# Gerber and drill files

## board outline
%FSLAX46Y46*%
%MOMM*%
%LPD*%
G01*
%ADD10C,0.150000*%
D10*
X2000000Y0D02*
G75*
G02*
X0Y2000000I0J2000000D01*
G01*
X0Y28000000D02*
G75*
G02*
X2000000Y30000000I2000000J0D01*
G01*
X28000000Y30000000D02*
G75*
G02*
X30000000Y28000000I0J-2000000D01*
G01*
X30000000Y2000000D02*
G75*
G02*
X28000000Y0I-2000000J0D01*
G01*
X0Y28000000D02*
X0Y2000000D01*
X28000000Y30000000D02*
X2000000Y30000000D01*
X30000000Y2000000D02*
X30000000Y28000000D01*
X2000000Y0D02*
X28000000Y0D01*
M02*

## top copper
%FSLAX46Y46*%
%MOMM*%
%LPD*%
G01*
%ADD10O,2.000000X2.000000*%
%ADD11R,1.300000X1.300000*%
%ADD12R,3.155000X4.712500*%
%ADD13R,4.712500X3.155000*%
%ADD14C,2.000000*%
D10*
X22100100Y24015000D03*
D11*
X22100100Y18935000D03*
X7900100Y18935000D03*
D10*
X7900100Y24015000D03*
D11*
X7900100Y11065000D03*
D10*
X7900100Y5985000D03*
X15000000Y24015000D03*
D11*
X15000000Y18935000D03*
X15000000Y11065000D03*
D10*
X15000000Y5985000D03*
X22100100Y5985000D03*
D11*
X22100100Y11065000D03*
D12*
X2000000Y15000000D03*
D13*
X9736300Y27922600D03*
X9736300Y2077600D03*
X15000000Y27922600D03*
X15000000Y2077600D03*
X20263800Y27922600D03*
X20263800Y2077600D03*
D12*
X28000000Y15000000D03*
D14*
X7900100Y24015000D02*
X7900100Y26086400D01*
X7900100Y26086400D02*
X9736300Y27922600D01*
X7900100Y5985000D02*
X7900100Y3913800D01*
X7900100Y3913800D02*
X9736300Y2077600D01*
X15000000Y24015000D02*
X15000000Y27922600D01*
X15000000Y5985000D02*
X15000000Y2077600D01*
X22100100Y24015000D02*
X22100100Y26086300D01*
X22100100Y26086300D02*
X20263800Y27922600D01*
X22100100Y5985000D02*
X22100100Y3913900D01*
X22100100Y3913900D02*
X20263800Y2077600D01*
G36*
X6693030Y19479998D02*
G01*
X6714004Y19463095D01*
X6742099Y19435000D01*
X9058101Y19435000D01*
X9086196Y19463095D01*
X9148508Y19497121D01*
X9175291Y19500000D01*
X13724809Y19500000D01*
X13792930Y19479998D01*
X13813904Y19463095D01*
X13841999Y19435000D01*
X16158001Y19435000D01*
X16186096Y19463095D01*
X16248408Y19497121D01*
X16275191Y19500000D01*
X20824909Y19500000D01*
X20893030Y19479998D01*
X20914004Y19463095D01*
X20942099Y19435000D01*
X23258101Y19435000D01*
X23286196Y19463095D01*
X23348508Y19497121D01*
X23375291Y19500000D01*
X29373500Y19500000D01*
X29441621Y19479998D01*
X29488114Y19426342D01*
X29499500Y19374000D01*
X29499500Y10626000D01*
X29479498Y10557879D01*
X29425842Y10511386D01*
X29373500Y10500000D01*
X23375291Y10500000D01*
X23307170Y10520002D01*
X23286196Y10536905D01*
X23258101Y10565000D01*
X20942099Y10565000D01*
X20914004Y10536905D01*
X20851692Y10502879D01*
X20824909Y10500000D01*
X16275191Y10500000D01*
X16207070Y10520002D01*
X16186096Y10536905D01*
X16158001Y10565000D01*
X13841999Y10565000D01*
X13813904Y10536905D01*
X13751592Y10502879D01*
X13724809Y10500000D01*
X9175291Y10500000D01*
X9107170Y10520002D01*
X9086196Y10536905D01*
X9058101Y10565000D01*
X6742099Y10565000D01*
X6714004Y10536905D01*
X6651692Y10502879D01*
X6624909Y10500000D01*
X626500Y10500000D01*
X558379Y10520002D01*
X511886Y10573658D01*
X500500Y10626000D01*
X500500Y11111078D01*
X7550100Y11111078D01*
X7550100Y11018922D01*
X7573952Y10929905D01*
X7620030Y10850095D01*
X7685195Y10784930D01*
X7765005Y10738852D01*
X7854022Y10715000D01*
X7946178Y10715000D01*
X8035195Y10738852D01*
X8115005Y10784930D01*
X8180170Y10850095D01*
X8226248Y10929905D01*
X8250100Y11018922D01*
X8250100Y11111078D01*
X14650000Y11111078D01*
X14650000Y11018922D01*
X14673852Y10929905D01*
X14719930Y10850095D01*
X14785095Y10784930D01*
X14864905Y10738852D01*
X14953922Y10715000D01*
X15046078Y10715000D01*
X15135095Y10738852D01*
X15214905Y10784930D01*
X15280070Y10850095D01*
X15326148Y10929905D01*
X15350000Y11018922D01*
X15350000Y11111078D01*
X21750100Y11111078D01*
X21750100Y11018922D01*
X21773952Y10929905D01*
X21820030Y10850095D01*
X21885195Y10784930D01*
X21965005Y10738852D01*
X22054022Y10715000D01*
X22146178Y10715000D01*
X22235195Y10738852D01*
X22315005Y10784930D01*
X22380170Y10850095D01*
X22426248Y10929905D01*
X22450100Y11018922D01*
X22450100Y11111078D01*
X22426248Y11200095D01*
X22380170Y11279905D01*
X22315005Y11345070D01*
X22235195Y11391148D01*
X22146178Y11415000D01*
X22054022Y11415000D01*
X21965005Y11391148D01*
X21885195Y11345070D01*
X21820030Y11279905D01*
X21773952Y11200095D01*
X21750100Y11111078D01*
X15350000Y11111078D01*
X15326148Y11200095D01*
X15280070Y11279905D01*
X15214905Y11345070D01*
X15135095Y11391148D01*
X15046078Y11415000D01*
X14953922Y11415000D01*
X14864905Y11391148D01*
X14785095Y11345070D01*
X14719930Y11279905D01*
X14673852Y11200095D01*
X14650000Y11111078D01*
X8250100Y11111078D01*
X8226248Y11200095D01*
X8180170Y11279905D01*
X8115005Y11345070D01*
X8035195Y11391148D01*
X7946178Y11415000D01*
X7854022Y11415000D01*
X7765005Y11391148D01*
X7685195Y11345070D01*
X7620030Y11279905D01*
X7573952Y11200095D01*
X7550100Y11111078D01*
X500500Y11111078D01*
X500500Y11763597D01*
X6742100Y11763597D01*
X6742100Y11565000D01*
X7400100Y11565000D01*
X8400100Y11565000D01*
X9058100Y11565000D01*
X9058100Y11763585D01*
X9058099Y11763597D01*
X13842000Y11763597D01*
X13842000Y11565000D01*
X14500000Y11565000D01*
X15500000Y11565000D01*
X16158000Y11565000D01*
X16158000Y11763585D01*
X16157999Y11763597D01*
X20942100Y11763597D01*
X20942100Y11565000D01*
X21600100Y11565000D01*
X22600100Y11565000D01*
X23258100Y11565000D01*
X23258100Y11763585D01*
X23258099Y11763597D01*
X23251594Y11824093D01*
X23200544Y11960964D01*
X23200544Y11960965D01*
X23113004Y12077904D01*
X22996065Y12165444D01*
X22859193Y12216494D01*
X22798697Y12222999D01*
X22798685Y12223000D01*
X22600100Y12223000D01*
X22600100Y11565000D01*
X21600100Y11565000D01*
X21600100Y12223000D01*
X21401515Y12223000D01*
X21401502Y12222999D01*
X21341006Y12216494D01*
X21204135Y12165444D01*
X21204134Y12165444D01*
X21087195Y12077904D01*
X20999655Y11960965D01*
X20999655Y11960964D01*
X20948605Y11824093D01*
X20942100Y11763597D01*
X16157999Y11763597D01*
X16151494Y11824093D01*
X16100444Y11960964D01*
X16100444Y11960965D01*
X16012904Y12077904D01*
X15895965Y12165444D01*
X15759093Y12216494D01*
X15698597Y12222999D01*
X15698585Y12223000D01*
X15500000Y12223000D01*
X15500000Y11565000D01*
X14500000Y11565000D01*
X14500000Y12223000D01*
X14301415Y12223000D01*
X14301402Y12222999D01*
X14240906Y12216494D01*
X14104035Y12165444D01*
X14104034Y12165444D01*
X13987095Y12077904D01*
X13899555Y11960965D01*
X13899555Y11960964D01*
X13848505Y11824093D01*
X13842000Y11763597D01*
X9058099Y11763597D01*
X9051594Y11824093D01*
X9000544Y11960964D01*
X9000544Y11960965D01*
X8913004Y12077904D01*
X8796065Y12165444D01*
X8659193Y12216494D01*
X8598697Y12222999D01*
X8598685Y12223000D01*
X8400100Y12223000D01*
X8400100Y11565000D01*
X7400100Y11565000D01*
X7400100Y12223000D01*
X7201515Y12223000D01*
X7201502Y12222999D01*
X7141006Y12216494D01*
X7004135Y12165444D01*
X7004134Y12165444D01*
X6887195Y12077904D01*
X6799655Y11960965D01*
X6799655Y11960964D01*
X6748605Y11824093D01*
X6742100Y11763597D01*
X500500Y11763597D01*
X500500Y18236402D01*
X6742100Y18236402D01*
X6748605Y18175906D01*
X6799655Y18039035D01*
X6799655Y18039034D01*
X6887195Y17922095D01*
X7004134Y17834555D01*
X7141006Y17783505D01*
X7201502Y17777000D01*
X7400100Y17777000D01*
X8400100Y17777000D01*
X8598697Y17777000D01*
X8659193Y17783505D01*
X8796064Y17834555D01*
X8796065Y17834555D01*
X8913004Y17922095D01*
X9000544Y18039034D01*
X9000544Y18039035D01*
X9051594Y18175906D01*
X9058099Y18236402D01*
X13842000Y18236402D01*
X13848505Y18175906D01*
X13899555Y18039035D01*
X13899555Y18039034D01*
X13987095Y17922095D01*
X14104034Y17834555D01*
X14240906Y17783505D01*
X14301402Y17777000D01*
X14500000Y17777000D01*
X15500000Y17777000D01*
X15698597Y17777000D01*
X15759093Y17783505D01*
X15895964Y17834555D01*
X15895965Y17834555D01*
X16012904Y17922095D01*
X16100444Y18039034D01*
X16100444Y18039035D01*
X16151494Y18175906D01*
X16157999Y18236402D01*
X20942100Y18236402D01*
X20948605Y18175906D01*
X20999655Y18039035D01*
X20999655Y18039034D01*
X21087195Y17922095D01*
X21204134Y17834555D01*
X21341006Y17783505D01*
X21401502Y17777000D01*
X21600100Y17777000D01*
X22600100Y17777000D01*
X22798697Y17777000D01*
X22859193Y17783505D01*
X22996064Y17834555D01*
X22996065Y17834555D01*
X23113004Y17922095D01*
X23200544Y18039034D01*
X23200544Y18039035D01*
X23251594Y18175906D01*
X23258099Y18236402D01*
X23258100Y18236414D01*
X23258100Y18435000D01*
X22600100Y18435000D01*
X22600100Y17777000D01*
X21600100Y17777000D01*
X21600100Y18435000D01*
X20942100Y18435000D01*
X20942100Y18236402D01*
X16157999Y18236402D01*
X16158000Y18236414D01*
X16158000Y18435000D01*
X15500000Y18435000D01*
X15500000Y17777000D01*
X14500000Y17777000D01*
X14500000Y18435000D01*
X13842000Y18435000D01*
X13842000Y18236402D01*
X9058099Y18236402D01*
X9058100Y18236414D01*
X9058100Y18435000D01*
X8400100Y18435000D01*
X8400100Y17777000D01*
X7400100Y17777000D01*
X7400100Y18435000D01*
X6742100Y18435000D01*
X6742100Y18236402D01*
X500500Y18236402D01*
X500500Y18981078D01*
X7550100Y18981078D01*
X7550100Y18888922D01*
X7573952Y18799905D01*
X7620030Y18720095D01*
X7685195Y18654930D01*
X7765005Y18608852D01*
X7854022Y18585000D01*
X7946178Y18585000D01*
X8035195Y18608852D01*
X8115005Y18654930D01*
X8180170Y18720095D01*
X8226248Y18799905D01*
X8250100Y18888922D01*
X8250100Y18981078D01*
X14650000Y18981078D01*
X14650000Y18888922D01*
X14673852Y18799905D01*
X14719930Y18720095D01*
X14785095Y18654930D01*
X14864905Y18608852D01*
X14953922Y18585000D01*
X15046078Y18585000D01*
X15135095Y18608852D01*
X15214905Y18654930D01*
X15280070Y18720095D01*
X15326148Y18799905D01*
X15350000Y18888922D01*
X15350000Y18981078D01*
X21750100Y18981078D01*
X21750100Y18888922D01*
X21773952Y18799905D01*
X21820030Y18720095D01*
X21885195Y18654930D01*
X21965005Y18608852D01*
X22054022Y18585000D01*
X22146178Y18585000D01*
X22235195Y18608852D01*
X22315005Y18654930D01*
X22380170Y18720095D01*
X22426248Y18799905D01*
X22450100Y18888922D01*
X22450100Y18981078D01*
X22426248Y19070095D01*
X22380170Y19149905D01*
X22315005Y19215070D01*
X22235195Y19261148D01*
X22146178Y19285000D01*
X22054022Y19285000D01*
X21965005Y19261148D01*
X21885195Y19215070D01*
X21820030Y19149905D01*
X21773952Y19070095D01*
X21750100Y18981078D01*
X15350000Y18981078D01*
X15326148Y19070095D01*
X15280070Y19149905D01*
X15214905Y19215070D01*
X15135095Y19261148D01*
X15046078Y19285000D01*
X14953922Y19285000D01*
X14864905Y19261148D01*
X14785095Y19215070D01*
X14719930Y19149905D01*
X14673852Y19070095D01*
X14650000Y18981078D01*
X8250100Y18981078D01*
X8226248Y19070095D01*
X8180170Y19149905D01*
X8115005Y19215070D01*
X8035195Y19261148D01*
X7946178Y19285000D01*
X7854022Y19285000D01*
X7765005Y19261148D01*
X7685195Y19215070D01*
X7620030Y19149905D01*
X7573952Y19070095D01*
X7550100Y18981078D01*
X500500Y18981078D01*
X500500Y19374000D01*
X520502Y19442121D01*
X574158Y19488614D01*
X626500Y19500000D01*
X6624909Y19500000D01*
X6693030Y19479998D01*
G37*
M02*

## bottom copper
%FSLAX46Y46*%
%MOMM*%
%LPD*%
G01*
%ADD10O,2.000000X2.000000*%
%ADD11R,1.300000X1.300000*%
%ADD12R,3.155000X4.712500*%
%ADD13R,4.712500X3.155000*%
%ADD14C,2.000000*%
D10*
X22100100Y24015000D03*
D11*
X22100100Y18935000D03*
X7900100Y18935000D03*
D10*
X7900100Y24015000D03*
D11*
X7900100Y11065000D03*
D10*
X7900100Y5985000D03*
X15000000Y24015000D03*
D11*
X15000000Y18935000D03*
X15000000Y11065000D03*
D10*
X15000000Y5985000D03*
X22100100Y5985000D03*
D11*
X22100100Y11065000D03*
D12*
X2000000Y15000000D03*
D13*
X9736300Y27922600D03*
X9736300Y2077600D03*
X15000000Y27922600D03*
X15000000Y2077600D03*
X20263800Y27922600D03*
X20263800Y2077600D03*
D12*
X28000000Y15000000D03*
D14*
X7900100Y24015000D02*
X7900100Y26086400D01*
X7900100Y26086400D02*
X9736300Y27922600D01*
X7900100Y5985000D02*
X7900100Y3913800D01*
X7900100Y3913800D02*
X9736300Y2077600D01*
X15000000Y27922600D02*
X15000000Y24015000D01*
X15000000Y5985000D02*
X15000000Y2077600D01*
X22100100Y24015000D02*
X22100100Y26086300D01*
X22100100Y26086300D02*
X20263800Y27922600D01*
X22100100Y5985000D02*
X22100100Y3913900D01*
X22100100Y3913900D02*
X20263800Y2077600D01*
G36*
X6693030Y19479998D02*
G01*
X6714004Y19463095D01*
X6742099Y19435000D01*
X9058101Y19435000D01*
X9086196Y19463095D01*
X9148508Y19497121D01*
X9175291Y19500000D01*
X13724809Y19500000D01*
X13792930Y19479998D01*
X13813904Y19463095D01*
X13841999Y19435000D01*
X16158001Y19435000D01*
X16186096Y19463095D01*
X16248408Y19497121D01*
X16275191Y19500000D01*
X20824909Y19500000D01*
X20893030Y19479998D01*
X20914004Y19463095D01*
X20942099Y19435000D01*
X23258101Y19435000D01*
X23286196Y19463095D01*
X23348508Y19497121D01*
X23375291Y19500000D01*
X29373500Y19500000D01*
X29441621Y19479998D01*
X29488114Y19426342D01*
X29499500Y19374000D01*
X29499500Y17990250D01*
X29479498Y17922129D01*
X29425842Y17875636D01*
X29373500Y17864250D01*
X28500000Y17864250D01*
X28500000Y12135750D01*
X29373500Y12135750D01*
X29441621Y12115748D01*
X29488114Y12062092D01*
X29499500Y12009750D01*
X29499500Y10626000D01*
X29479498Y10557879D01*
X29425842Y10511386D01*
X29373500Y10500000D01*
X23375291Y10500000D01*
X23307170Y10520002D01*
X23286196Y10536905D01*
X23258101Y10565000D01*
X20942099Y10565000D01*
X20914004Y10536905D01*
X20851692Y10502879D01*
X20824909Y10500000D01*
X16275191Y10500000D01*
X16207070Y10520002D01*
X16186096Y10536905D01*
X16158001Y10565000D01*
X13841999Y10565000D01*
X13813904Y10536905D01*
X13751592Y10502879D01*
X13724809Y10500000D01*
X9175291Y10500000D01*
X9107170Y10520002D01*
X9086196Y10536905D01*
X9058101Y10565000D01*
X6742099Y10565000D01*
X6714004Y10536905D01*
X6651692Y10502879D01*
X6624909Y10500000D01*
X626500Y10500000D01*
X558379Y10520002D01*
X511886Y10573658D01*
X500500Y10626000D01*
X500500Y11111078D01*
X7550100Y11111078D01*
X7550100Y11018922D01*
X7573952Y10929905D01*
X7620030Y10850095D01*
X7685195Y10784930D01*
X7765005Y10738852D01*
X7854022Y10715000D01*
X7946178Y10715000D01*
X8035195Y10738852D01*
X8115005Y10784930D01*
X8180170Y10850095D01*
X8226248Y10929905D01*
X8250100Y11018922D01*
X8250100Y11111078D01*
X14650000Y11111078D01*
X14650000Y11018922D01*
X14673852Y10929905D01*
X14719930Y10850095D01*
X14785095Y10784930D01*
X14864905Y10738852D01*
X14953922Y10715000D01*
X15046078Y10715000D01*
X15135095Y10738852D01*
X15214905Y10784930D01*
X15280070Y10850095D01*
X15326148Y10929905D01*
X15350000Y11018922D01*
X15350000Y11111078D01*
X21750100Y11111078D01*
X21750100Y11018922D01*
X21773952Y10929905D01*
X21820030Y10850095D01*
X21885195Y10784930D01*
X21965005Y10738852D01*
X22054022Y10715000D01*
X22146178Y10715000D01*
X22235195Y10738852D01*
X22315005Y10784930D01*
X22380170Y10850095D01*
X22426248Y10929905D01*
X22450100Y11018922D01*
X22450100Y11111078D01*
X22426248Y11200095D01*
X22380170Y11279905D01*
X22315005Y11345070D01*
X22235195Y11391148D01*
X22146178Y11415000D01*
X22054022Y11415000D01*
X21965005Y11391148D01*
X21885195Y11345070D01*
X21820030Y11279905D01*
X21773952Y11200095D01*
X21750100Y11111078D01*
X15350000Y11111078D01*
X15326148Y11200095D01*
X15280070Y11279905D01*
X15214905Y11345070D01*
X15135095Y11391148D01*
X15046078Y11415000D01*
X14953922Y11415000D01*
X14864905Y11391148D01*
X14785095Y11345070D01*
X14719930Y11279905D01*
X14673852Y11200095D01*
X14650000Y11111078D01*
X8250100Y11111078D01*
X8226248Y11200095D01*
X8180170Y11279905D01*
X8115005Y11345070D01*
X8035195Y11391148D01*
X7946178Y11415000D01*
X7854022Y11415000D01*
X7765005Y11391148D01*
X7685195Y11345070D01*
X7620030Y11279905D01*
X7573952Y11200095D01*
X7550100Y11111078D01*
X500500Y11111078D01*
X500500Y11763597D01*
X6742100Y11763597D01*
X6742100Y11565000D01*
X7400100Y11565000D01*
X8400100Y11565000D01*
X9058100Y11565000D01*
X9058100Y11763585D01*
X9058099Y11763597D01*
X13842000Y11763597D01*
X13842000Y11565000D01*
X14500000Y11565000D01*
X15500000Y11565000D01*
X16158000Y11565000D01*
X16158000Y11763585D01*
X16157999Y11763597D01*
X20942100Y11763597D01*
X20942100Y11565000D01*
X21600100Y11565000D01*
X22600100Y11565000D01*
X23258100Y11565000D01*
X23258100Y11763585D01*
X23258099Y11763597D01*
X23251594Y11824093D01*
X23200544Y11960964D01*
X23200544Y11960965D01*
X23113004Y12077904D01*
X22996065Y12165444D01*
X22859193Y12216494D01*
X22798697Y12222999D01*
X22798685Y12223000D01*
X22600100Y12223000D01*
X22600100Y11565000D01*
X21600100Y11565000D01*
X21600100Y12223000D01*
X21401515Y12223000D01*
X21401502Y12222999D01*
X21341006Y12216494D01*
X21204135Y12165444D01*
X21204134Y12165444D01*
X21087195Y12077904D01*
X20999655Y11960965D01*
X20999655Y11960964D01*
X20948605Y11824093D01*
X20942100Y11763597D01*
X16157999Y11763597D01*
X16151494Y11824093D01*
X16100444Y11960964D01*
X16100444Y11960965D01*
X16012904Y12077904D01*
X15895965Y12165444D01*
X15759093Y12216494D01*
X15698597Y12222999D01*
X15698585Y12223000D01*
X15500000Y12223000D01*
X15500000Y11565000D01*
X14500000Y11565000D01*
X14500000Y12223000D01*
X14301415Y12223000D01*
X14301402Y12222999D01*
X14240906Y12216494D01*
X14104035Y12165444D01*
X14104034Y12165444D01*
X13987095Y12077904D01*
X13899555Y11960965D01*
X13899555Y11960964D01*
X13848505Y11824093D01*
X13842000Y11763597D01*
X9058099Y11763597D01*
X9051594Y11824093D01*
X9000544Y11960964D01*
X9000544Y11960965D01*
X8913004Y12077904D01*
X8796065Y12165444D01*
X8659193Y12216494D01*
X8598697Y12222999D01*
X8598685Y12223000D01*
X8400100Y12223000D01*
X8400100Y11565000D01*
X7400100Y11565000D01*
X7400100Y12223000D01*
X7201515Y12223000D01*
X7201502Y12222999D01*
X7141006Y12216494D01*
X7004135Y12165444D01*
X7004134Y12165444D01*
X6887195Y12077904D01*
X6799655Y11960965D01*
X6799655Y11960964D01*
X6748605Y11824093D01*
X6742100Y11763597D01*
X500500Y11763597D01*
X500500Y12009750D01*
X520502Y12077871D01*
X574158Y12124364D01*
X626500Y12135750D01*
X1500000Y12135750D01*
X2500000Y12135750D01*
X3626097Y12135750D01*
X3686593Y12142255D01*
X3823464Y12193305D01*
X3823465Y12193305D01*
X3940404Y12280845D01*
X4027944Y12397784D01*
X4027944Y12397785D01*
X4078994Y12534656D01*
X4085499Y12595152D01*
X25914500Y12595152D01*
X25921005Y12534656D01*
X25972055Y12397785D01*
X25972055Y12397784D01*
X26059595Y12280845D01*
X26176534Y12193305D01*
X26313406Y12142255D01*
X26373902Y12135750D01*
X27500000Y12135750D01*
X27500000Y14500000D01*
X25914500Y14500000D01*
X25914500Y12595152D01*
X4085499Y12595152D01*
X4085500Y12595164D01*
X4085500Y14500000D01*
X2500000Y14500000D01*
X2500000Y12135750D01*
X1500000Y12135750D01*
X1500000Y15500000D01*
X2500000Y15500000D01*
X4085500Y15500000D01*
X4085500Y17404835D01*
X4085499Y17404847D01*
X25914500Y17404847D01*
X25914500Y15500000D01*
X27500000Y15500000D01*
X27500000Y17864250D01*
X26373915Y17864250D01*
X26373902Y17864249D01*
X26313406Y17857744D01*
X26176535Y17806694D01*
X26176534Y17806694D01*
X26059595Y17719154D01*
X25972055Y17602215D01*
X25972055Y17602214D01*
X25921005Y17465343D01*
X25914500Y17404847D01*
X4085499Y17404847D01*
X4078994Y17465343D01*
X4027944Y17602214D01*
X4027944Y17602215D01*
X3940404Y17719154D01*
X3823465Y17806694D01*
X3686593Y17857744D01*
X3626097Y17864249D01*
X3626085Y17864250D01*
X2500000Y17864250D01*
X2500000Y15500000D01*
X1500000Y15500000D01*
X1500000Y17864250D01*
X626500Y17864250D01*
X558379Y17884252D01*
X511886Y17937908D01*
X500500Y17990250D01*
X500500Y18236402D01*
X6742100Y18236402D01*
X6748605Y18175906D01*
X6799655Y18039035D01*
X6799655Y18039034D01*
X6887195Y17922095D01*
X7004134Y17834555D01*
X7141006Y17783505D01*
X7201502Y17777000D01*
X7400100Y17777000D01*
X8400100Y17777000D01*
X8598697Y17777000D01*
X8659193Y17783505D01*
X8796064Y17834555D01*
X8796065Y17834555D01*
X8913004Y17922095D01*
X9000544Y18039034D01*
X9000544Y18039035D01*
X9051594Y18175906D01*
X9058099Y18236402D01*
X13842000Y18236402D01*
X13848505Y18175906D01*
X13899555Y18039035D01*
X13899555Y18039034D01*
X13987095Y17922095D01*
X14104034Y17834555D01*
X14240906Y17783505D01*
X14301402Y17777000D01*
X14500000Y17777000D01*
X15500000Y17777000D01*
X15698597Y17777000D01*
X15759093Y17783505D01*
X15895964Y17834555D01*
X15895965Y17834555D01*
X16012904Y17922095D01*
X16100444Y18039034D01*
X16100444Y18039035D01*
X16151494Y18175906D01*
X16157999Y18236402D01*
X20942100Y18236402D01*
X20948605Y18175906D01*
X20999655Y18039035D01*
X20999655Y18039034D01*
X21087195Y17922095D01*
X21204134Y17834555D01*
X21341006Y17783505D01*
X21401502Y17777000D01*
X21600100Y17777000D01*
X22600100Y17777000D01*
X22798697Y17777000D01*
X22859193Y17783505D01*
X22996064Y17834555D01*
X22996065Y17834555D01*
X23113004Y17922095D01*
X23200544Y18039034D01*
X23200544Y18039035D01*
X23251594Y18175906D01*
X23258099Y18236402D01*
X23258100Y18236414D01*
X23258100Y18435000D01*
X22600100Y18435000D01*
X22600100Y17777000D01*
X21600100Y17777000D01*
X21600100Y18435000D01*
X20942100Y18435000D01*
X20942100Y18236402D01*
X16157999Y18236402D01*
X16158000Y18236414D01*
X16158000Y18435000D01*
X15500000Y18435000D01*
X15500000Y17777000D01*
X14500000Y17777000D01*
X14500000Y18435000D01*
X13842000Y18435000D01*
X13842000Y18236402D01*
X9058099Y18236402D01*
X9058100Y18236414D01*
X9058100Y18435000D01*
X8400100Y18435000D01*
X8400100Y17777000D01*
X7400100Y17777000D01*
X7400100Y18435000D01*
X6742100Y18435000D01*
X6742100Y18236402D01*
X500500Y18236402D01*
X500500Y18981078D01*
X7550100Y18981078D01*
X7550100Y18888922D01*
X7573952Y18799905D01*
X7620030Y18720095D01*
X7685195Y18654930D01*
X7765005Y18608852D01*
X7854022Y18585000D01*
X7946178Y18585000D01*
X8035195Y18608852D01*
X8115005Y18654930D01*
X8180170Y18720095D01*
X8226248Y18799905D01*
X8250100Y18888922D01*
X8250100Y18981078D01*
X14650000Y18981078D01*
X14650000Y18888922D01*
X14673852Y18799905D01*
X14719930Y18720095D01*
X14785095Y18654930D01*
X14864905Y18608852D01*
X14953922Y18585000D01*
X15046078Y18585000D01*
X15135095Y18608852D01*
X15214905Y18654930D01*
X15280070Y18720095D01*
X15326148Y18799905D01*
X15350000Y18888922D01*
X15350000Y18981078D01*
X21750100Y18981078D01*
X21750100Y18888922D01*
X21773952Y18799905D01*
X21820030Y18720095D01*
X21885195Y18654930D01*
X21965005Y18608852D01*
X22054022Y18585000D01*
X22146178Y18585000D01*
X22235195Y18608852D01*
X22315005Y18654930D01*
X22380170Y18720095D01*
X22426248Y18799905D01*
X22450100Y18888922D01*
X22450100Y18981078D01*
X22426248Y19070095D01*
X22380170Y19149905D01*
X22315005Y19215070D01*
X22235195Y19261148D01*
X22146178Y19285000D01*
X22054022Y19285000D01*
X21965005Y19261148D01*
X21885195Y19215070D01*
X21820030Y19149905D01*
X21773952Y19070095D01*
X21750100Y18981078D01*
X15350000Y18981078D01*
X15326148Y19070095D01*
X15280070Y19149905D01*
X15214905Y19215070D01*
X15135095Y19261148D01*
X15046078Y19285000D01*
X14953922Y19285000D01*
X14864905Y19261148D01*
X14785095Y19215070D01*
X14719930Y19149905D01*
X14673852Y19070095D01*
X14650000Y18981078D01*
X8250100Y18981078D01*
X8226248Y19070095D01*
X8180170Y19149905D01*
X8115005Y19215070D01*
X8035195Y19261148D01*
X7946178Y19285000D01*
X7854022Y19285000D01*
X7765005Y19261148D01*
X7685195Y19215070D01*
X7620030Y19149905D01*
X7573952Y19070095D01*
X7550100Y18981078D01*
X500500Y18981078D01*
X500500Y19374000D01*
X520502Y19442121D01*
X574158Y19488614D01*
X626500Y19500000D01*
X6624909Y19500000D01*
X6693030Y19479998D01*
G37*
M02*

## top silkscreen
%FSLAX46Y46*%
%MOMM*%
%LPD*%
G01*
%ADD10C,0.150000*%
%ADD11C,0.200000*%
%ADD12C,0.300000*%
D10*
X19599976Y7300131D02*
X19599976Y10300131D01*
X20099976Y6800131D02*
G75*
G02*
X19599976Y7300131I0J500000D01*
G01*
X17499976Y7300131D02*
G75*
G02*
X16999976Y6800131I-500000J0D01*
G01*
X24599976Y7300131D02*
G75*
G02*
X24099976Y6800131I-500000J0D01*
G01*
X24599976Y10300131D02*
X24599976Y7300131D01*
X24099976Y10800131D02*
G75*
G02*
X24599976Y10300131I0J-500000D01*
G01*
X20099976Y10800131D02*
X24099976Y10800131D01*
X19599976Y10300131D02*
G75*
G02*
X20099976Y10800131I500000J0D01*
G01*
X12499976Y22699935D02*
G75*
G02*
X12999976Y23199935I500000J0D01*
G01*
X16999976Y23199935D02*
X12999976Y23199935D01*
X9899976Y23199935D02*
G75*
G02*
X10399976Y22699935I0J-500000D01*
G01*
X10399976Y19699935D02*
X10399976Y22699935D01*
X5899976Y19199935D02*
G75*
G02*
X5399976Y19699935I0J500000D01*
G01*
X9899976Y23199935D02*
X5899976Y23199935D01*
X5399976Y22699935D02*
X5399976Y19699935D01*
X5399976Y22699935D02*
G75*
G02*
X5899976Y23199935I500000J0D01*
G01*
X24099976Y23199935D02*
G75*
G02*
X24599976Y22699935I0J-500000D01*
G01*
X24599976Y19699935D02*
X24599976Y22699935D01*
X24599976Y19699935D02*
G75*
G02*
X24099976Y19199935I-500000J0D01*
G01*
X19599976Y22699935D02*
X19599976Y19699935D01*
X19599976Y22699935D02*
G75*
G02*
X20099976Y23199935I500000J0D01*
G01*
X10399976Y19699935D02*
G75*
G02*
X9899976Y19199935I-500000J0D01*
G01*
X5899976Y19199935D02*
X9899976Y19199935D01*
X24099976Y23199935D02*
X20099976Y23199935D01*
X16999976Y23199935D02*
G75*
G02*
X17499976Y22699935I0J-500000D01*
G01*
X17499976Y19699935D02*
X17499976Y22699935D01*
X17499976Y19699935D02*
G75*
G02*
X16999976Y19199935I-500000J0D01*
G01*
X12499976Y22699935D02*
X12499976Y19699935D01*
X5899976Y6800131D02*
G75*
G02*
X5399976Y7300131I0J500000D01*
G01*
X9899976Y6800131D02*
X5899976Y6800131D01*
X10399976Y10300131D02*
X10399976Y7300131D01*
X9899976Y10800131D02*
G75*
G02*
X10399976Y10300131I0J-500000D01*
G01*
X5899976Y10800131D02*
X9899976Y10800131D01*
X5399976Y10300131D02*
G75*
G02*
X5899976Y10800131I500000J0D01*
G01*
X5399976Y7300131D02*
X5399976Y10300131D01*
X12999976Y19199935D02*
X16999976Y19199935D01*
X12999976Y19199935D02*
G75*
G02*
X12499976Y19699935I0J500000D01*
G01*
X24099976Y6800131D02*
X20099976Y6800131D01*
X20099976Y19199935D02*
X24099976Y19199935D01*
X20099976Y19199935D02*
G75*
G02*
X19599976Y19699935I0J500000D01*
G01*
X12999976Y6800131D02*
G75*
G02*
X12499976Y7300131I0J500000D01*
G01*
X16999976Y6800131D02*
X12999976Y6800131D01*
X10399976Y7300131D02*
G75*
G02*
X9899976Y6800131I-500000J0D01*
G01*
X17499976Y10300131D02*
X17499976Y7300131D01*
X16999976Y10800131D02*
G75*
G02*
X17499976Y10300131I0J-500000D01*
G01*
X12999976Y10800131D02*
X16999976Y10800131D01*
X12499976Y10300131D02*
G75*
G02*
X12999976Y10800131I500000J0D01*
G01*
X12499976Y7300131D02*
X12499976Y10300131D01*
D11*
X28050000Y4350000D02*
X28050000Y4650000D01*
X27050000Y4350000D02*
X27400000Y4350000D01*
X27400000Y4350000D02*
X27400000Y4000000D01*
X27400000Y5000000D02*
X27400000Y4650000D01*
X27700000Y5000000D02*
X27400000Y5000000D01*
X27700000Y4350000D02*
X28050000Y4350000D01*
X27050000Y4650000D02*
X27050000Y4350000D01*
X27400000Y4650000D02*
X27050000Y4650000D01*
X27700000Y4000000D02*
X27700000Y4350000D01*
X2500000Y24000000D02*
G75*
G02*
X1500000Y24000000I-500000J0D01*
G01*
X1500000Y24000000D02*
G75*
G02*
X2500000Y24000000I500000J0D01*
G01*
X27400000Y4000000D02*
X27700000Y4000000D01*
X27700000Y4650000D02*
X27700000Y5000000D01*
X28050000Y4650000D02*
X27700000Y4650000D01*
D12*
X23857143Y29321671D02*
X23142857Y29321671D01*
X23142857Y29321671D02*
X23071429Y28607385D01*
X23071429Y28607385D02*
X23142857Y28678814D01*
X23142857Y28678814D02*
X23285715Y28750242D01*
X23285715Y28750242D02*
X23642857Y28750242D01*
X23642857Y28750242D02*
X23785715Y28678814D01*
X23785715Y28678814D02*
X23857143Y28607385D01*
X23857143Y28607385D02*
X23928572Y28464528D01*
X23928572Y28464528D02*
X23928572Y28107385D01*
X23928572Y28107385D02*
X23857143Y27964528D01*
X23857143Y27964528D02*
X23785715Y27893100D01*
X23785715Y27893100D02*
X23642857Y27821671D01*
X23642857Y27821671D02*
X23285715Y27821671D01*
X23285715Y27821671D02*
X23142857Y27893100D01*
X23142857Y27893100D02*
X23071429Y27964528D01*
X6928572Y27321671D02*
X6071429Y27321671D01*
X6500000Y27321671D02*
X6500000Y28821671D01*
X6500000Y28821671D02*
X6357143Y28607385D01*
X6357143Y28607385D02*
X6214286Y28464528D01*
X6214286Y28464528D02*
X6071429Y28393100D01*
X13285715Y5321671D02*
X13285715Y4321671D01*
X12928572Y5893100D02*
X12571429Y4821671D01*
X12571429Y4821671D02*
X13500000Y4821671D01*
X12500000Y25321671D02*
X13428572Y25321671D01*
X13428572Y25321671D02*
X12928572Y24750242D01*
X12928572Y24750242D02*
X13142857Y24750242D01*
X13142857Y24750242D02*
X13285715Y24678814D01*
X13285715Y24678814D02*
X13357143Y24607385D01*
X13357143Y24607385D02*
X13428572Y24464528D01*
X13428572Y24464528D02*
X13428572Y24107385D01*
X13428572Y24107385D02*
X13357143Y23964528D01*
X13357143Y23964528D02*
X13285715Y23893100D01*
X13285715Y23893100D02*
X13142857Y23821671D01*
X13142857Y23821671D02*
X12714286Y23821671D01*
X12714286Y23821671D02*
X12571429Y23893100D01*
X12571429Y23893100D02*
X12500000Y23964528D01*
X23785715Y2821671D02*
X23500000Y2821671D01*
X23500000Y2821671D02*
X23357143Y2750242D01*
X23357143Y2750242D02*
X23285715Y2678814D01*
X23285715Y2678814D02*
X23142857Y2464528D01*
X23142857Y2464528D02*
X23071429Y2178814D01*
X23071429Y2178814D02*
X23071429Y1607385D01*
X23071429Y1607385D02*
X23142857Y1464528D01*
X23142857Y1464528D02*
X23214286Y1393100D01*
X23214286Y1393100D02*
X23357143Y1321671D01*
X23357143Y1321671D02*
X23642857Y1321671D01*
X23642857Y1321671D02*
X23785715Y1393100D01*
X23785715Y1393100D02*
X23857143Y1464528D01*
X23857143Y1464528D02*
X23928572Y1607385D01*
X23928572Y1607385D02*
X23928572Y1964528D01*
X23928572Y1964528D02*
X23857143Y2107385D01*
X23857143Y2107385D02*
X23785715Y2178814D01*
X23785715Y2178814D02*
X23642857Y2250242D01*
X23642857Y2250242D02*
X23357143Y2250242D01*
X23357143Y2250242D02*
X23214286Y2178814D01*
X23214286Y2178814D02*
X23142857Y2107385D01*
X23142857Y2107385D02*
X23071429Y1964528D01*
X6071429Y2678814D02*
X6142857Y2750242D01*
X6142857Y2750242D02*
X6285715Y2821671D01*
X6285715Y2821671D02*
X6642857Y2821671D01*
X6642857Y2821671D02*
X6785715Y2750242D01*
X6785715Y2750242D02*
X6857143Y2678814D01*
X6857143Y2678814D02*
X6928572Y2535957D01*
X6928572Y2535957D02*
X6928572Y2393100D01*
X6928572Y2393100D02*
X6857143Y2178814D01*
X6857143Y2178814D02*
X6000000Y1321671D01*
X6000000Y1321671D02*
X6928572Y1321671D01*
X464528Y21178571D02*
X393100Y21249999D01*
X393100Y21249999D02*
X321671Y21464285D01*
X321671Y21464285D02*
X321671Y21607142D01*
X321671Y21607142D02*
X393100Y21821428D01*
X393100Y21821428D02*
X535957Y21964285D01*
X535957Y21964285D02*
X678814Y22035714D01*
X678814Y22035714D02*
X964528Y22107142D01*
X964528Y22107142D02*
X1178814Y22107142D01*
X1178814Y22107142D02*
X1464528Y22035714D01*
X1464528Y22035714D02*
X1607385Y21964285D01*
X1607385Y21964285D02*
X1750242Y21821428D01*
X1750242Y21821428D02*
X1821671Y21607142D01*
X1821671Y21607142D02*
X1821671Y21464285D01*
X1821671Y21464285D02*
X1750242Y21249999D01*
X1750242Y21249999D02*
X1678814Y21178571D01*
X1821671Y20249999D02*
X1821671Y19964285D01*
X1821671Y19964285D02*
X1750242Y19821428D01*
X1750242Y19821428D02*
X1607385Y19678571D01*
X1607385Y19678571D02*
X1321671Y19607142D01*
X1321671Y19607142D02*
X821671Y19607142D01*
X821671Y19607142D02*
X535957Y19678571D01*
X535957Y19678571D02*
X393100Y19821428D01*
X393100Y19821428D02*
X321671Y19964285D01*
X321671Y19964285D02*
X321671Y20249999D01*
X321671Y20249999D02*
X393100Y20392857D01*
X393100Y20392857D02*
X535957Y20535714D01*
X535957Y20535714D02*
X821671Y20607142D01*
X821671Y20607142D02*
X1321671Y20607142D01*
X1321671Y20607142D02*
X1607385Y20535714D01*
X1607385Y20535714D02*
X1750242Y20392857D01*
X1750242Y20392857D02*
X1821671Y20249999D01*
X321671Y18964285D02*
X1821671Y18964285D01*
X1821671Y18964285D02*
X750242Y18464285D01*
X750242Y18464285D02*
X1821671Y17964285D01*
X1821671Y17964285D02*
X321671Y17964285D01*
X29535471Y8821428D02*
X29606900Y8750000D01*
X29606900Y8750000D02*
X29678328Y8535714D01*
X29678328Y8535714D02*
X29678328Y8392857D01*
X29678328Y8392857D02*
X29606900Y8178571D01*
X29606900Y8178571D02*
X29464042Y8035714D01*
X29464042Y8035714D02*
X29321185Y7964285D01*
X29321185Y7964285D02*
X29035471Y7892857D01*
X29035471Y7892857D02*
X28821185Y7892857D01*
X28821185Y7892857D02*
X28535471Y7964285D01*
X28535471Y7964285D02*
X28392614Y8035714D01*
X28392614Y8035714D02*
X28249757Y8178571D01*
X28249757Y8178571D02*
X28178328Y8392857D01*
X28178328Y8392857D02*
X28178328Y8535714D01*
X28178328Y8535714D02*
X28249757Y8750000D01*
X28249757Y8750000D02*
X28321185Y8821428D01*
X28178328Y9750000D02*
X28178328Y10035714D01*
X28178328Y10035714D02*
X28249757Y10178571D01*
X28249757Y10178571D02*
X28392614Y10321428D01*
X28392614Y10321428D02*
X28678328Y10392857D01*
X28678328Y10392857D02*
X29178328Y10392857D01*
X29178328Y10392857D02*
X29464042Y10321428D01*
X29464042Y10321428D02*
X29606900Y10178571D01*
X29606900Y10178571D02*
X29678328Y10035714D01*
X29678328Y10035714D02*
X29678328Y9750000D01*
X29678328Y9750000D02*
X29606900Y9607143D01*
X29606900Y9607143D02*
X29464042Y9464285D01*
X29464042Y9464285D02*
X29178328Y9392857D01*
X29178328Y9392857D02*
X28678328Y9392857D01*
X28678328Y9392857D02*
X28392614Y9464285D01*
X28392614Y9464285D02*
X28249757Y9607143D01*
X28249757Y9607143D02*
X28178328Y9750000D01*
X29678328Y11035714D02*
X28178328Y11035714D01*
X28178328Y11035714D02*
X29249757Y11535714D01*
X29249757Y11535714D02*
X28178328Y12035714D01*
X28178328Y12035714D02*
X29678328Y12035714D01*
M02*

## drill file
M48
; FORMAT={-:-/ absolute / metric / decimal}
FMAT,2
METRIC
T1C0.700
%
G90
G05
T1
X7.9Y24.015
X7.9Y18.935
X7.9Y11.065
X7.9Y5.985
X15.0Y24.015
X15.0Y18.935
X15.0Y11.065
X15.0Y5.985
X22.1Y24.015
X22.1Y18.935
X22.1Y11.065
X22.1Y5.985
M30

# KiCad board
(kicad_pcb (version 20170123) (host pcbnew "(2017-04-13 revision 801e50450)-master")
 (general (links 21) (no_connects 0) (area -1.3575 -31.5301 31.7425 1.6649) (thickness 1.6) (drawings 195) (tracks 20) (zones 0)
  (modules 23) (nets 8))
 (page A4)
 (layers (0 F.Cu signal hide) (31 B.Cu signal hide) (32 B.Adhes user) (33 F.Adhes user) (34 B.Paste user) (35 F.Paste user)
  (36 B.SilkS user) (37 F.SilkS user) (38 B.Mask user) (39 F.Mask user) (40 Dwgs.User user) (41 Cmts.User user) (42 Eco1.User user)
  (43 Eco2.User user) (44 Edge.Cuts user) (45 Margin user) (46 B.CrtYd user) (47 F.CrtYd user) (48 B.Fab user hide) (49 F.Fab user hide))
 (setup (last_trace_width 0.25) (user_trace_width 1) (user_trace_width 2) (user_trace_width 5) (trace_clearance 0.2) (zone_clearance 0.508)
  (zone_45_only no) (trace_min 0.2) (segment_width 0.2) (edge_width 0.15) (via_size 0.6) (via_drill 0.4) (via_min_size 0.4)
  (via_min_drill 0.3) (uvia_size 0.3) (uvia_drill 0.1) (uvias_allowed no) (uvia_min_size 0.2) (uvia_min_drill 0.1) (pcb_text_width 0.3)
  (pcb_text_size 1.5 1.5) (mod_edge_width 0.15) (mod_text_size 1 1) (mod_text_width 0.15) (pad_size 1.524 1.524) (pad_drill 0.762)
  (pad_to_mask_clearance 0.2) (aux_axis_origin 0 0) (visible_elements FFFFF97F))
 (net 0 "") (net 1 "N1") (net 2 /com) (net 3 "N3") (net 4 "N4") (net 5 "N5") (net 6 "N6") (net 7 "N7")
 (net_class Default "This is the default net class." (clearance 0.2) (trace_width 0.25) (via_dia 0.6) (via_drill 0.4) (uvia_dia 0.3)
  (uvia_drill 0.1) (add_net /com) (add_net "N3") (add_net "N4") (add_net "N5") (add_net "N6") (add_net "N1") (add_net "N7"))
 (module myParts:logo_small (layer B.Cu) (at 15 -15)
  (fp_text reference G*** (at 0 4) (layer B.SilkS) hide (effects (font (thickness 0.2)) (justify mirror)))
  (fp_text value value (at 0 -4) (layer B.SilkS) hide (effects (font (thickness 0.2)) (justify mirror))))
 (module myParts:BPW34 (layer B.Cu) (at 22.1001 -18.935 90)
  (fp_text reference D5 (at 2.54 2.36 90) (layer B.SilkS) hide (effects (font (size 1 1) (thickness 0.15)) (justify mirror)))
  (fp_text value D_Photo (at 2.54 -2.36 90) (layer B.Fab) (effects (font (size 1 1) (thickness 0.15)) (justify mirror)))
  (pad 2 thru_hole oval (at 5.08 0 90) (size 2 2) (drill 0.7) (layers *.Cu *.Mask) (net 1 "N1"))
  (pad 1 thru_hole rect (at 0 0 90) (size 1.3 1.3) (drill 0.7) (layers *.Cu *.Mask) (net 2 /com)))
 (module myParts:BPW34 (layer B.Cu) (at 7.9001 -18.935 90)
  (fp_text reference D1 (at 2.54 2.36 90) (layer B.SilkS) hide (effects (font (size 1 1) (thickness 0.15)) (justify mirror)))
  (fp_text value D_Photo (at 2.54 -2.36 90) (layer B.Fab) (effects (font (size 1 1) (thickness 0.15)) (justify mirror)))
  (pad 1 thru_hole rect (at 0 0 90) (size 1.3 1.3) (drill 0.7) (layers *.Cu *.Mask) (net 2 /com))
  (pad 2 thru_hole oval (at 5.08 0 90) (size 2 2) (drill 0.7) (layers *.Cu *.Mask) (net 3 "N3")))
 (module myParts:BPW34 (layer B.Cu) (at 7.9001 -11.065 270)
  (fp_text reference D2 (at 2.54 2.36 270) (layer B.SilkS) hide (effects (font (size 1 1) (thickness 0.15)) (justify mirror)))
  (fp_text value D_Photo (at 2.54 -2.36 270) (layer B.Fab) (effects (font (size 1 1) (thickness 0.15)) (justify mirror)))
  (pad 1 thru_hole rect (at 0 0 270) (size 1.3 1.3) (drill 0.7) (layers *.Cu *.Mask) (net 2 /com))
  (pad 2 thru_hole oval (at 5.08 0 270) (size 2 2) (drill 0.7) (layers *.Cu *.Mask) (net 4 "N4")))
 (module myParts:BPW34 (layer B.Cu) (at 15 -18.935 90)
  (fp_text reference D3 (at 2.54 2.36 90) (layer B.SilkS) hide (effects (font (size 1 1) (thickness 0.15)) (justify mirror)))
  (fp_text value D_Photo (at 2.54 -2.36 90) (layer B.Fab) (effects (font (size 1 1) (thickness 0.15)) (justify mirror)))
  (pad 2 thru_hole oval (at 5.08 0 90) (size 2 2) (drill 0.7) (layers *.Cu *.Mask) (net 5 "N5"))
  (pad 1 thru_hole rect (at 0 0 90) (size 1.3 1.3) (drill 0.7) (layers *.Cu *.Mask) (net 2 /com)))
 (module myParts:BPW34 (layer B.Cu) (at 15 -11.065 270)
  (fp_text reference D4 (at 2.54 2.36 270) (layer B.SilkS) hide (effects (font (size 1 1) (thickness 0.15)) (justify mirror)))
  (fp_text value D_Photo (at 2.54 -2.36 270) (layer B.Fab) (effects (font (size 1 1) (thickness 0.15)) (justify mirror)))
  (pad 1 thru_hole rect (at 0 0 270) (size 1.3 1.3) (drill 0.7) (layers *.Cu *.Mask) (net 2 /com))
  (pad 2 thru_hole oval (at 5.08 0 270) (size 2 2) (drill 0.7) (layers *.Cu *.Mask) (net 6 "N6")))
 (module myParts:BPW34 (layer B.Cu) (at 22.1001 -11.065 270)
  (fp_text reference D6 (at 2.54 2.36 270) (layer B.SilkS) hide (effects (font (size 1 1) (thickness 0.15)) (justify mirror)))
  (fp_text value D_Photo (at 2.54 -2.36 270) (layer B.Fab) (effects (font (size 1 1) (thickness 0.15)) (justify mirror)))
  (pad 2 thru_hole oval (at 5.08 0 270) (size 2 2) (drill 0.7) (layers *.Cu *.Mask) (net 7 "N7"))
  (pad 1 thru_hole rect (at 0 0 270) (size 1.3 1.3) (drill 0.7) (layers *.Cu *.Mask) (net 2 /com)))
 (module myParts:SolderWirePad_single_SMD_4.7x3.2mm (layer F.Cu) (at 2 -15 90)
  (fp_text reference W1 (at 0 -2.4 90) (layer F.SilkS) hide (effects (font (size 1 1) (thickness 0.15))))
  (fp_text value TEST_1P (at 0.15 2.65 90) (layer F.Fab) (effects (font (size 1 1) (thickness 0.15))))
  (pad 1 smd rect (at 0 0 90) (size 4.7125 3.155) (layers F.Cu F.Paste F.Mask) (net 2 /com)))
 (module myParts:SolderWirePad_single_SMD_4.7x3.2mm (layer F.Cu) (at 9.7363 -27.9226)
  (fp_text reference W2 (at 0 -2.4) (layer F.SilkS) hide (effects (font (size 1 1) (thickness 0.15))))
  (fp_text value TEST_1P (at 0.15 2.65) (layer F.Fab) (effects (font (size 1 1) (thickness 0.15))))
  (pad 1 smd rect (at 0 0) (size 4.7125 3.155) (layers F.Cu F.Paste F.Mask) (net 3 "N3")))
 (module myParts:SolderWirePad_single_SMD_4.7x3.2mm (layer F.Cu) (at 9.7363 -2.0776)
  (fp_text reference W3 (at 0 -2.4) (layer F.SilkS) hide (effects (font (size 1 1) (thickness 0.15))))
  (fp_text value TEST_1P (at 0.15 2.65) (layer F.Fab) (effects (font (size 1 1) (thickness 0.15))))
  (pad 1 smd rect (at 0 0) (size 4.7125 3.155) (layers F.Cu F.Paste F.Mask) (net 4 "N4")))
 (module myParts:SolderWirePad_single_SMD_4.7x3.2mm (layer F.Cu) (at 15 -27.9226)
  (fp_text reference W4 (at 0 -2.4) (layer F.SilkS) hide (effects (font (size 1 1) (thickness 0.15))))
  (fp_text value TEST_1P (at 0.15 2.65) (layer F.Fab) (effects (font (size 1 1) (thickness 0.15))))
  (pad 1 smd rect (at 0 0) (size 4.7125 3.155) (layers F.Cu F.Paste F.Mask) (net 5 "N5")))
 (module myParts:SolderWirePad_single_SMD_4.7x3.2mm (layer F.Cu) (at 15 -2.0776)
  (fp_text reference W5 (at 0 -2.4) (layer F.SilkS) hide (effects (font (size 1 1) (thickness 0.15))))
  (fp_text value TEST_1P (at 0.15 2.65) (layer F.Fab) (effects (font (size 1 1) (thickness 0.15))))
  (pad 1 smd rect (at 0 0) (size 4.7125 3.155) (layers F.Cu F.Paste F.Mask) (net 6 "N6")))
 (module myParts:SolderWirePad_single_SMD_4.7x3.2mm (layer F.Cu) (at 20.2638 -27.9226)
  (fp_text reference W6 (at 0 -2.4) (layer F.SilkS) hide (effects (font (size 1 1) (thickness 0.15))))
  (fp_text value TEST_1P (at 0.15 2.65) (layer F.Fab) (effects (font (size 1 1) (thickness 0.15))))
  (pad 1 smd rect (at 0 0) (size 4.7125 3.155) (layers F.Cu F.Paste F.Mask) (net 1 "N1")))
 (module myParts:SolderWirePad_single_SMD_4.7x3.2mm (layer F.Cu) (at 20.2638 -2.0776)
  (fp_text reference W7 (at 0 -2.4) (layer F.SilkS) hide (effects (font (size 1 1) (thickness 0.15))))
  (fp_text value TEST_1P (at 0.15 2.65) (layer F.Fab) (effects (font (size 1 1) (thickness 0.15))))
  (pad 1 smd rect (at 0 0) (size 4.7125 3.155) (layers F.Cu F.Paste F.Mask) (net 7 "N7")))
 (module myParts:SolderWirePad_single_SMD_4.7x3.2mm (layer F.Cu) (at 28 -15 90)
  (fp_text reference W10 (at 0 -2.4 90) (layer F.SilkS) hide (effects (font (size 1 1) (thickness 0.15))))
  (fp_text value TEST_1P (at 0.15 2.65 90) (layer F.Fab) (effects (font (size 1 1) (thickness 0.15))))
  (pad 1 smd rect (at 0 0 90) (size 4.7125 3.155) (layers F.Cu F.Paste F.Mask) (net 2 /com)))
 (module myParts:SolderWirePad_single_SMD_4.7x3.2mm (layer B.Cu) (at 2 -15 270)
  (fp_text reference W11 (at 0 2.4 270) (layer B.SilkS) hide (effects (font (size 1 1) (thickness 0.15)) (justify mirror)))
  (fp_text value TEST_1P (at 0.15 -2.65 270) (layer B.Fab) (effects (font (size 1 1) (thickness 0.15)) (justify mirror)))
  (pad 1 smd rect (at 0 0 270) (size 4.7125 3.155) (layers B.Cu B.Paste B.Mask) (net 2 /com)))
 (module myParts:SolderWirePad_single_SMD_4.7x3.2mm (layer B.Cu) (at 9.7363 -27.9226)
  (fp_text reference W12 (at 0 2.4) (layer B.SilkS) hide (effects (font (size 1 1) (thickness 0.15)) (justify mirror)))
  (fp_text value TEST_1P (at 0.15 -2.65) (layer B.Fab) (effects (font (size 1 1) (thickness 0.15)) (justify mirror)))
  (pad 1 smd rect (at 0 0) (size 4.7125 3.155) (layers B.Cu B.Paste B.Mask) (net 3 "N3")))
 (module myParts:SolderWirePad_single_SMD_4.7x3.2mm (layer B.Cu) (at 9.7363 -2.0776)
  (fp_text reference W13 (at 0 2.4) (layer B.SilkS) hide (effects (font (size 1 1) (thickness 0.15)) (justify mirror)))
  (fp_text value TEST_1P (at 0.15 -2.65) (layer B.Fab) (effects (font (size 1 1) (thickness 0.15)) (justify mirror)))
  (pad 1 smd rect (at 0 0) (size 4.7125 3.155) (layers B.Cu B.Paste B.Mask) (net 4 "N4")))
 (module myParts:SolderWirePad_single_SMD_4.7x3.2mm (layer B.Cu) (at 15 -27.9226)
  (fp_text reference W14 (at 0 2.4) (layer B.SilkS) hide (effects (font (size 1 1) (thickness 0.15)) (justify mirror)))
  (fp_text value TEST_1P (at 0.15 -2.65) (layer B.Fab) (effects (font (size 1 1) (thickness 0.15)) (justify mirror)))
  (pad 1 smd rect (at 0 0) (size 4.7125 3.155) (layers B.Cu B.Paste B.Mask) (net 5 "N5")))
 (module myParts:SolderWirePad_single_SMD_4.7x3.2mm (layer B.Cu) (at 15 -2.0776)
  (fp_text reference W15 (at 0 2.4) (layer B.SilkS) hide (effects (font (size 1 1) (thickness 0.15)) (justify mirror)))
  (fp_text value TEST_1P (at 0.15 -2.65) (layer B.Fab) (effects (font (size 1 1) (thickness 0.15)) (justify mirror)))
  (pad 1 smd rect (at 0 0) (size 4.7125 3.155) (layers B.Cu B.Paste B.Mask) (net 6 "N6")))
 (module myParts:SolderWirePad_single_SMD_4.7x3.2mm (layer B.Cu) (at 20.2638 -27.9226)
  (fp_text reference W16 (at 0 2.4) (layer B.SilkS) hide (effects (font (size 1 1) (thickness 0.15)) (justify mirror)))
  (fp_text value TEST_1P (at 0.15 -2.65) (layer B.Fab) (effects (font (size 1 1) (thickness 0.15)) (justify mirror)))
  (pad 1 smd rect (at 0 0) (size 4.7125 3.155) (layers B.Cu B.Paste B.Mask) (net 1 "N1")))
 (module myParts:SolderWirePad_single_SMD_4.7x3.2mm (layer B.Cu) (at 20.2638 -2.0776)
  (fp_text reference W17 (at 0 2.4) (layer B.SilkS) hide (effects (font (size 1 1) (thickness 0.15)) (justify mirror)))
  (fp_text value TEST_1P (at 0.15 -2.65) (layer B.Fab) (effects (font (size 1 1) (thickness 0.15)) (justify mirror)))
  (pad 1 smd rect (at 0 0) (size 4.7125 3.155) (layers B.Cu B.Paste B.Mask) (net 7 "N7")))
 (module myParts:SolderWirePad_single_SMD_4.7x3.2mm (layer B.Cu) (at 28 -15 270)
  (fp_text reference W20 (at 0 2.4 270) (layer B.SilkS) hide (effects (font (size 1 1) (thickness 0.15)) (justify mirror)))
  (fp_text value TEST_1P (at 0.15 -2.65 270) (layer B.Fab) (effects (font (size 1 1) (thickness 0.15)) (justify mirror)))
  (pad 1 smd rect (at 0 0 270) (size 4.7125 3.155) (layers B.Cu B.Paste B.Mask) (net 2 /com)))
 (gr_line (start 19.599976 -7.300131) (end 19.599976 -10.300131) (layer F.SilkS) (width 0.15))
 (gr_arc (start 20.099976 -7.300131) (end 19.599976 -7.300131) (angle -90) (layer F.SilkS) (width 0.15))
 (gr_arc (start 16.999976 -7.300131) (end 16.999976 -6.800131) (angle -90) (layer F.SilkS) (width 0.15))
 (gr_arc (start 24.099976 -7.300131) (end 24.099976 -6.800131) (angle -90) (layer F.SilkS) (width 0.15))
 (gr_line (start 24.599976 -10.300131) (end 24.599976 -7.300131) (layer F.SilkS) (width 0.15))
 (gr_arc (start 24.099976 -10.300131) (end 24.599976 -10.300131) (angle -90) (layer F.SilkS) (width 0.15))
 (gr_line (start 20.099976 -10.800131) (end 24.099976 -10.800131) (layer F.SilkS) (width 0.15))
 (gr_arc (start 20.099976 -10.300131) (end 20.099976 -10.800131) (angle -90) (layer F.SilkS) (width 0.15))
 (gr_arc (start 12.999976 -22.699935) (end 12.999976 -23.199935) (angle -90) (layer F.SilkS) (width 0.15))
 (gr_line (start 16.999976 -23.199935) (end 12.999976 -23.199935) (layer F.SilkS) (width 0.15))
 (gr_arc (start 9.899976 -22.699935) (end 10.399976 -22.699935) (angle -90) (layer F.SilkS) (width 0.15))
 (gr_line (start 10.399976 -19.699935) (end 10.399976 -22.699935) (layer F.SilkS) (width 0.15))
 (gr_arc (start 5.899976 -19.699935) (end 5.399976 -19.699935) (angle -90) (layer F.SilkS) (width 0.15))
 (gr_line (start 9.899976 -23.199935) (end 5.899976 -23.199935) (layer F.SilkS) (width 0.15))
 (gr_line (start 5.399976 -22.699935) (end 5.399976 -19.699935) (layer F.SilkS) (width 0.15))
 (gr_arc (start 5.899976 -22.699935) (end 5.899976 -23.199935) (angle -90) (layer F.SilkS) (width 0.15))
 (gr_arc (start 24.099976 -22.699935) (end 24.599976 -22.699935) (angle -90) (layer F.SilkS) (width 0.15))
 (gr_line (start 24.599976 -19.699935) (end 24.599976 -22.699935) (layer F.SilkS) (width 0.15))
 (gr_arc (start 24.099976 -19.699935) (end 24.099976 -19.199935) (angle -90) (layer F.SilkS) (width 0.15))
 (gr_line (start 19.599976 -22.699935) (end 19.599976 -19.699935) (layer F.SilkS) (width 0.15))
 (gr_arc (start 20.099976 -22.699935) (end 20.099976 -23.199935) (angle -90) (layer F.SilkS) (width 0.15))
 (gr_arc (start 9.899976 -19.699935) (end 9.899976 -19.199935) (angle -90) (layer F.SilkS) (width 0.15))
 (gr_line (start 5.899976 -19.199935) (end 9.899976 -19.199935) (layer F.SilkS) (width 0.15))
 (gr_line (start 24.099976 -23.199935) (end 20.099976 -23.199935) (layer F.SilkS) (width 0.15))
 (gr_arc (start 16.999976 -22.699935) (end 17.499976 -22.699935) (angle -90) (layer F.SilkS) (width 0.15))
 (gr_line (start 17.499976 -19.699935) (end 17.499976 -22.699935) (layer F.SilkS) (width 0.15))
 (gr_arc (start 16.999976 -19.699935) (end 16.999976 -19.199935) (angle -90) (layer F.SilkS) (width 0.15))
 (gr_line (start 12.499976 -22.699935) (end 12.499976 -19.699935) (layer F.SilkS) (width 0.15))
 (gr_arc (start 5.899976 -7.300131) (end 5.399976 -7.300131) (angle -90) (layer F.SilkS) (width 0.15))
 (gr_line (start 9.899976 -6.800131) (end 5.899976 -6.800131) (layer F.SilkS) (width 0.15))
 (gr_line (start 10.399976 -10.300131) (end 10.399976 -7.300131) (layer F.SilkS) (width 0.15))
 (gr_arc (start 9.899976 -10.300131) (end 10.399976 -10.300131) (angle -90) (layer F.SilkS) (width 0.15))
 (gr_line (start 5.899976 -10.800131) (end 9.899976 -10.800131) (layer F.SilkS) (width 0.15))
 (gr_arc (start 5.899976 -10.300131) (end 5.899976 -10.800131) (angle -90) (layer F.SilkS) (width 0.15))
 (gr_line (start 5.399976 -7.300131) (end 5.399976 -10.300131) (layer F.SilkS) (width 0.15))
 (gr_line (start 12.999976 -19.199935) (end 16.999976 -19.199935) (layer F.SilkS) (width 0.15))
 (gr_arc (start 12.999976 -19.699935) (end 12.499976 -19.699935) (angle -90) (layer F.SilkS) (width 0.15))
 (gr_line (start 24.099976 -6.800131) (end 20.099976 -6.800131) (layer F.SilkS) (width 0.15))
 (gr_line (start 20.099976 -19.199935) (end 24.099976 -19.199935) (layer F.SilkS) (width 0.15))
 (gr_arc (start 20.099976 -19.699935) (end 19.599976 -19.699935) (angle -90) (layer F.SilkS) (width 0.15))
 (gr_arc (start 12.999976 -7.300131) (end 12.499976 -7.300131) (angle -90) (layer F.SilkS) (width 0.15))
 (gr_line (start 16.999976 -6.800131) (end 12.999976 -6.800131) (layer F.SilkS) (width 0.15))
 (gr_arc (start 9.899976 -7.300131) (end 9.899976 -6.800131) (angle -90) (layer F.SilkS) (width 0.15))
 (gr_line (start 17.499976 -10.300131) (end 17.499976 -7.300131) (layer F.SilkS) (width 0.15))
 (gr_arc (start 16.999976 -10.300131) (end 17.499976 -10.300131) (angle -90) (layer F.SilkS) (width 0.15))
 (gr_line (start 12.999976 -10.800131) (end 16.999976 -10.800131) (layer F.SilkS) (width 0.15))
 (gr_arc (start 12.999976 -10.300131) (end 12.999976 -10.800131) (angle -90) (layer F.SilkS) (width 0.15))
 (gr_line (start 12.499976 -7.300131) (end 12.499976 -10.300131) (layer F.SilkS) (width 0.15))
 (gr_line (start 28.05 -4.35) (end 28.05 -4.65) (layer F.SilkS) (width 0.2))
 (gr_line (start 27.05 -4.35) (end 27.4 -4.35) (layer F.SilkS) (width 0.2))
 (gr_line (start 27.4 -4.35) (end 27.4 -4) (layer F.SilkS) (width 0.2))
 (gr_line (start 27.4 -5) (end 27.4 -4.65) (layer F.SilkS) (width 0.2))
 (gr_line (start 27.7 -5) (end 27.4 -5) (layer F.SilkS) (width 0.2))
 (gr_line (start 27.7 -4.35) (end 28.05 -4.35) (layer F.SilkS) (width 0.2))
 (gr_line (start 27.05 -4.65) (end 27.05 -4.35) (layer F.SilkS) (width 0.2))
 (gr_line (start 27.4 -4.65) (end 27.05 -4.65) (layer F.SilkS) (width 0.2))
 (gr_line (start 27.7 -4) (end 27.7 -4.35) (layer F.SilkS) (width 0.2))
 (gr_circle (center 2 -24) (end 2.5 -24) (layer F.SilkS) (width 0.2))
 (gr_line (start 27.4 -4) (end 27.7 -4) (layer F.SilkS) (width 0.2))
 (gr_line (start 27.7 -4.65) (end 27.7 -5) (layer F.SilkS) (width 0.2))
 (gr_line (start 28.05 -4.65) (end 27.7 -4.65) (layer F.SilkS) (width 0.2))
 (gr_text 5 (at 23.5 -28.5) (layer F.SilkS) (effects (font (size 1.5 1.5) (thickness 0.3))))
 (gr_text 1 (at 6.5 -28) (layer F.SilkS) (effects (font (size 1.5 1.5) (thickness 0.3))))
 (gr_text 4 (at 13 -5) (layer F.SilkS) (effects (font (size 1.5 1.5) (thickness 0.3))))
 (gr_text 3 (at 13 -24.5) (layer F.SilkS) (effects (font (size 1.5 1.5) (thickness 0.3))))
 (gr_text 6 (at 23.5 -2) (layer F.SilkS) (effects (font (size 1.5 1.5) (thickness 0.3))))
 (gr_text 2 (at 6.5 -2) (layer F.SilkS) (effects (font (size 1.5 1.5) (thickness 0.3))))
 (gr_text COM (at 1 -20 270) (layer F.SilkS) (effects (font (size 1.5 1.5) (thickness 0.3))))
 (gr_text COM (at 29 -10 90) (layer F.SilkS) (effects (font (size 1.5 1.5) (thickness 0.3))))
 (gr_arc (start 2 -2) (end 2 0) (angle 90) (layer Edge.Cuts) (width 0.15))
 (gr_arc (start 2 -28) (end 0 -28) (angle 90) (layer Edge.Cuts) (width 0.15))
 (gr_arc (start 28 -28) (end 28 -30) (angle 90) (layer Edge.Cuts) (width 0.15))
 (gr_arc (start 28 -2) (end 30 -2) (angle 90) (layer Edge.Cuts) (width 0.15))
 (gr_line (start 0 -28) (end 0 -2) (layer Edge.Cuts) (width 0.15))
 (gr_line (start 28 -30) (end 2 -30) (layer Edge.Cuts) (width 0.15))
 (gr_line (start 30 -2) (end 30 -28) (layer Edge.Cuts) (width 0.15))
 (gr_line (start 2 0) (end 28 0) (layer Edge.Cuts) (width 0.15))
 (segment (start 7.9001 -24.015) (end 7.9001 -26.0864) (width 2) (layer F.Cu) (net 3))
 (segment (start 7.9001 -26.0864) (end 9.7363 -27.9226) (width 2) (layer F.Cu) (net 3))
 (segment (start 7.9001 -24.015) (end 7.9001 -26.0864) (width 2) (layer B.Cu) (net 3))
 (segment (start 7.9001 -26.0864) (end 9.7363 -27.9226) (width 2) (layer B.Cu) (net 3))
 (segment (start 7.9001 -5.985) (end 7.9001 -3.9138) (width 2) (layer B.Cu) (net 4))
 (segment (start 7.9001 -3.9138) (end 9.7363 -2.0776) (width 2) (layer B.Cu) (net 4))
 (segment (start 7.9001 -5.985) (end 7.9001 -3.9138) (width 2) (layer F.Cu) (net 4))
 (segment (start 7.9001 -3.9138) (end 9.7363 -2.0776) (width 2) (layer F.Cu) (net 4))
 (segment (start 15 -24.015) (end 15 -27.9226) (width 2) (layer F.Cu) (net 5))
 (segment (start 15 -27.9226) (end 15 -24.015) (width 2) (layer B.Cu) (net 5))
 (segment (start 15 -5.985) (end 15 -2.0776) (width 2) (layer B.Cu) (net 6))
 (segment (start 15 -5.985) (end 15 -2.0776) (width 2) (layer F.Cu) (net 6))
 (segment (start 22.1001 -24.015) (end 22.1001 -26.0863) (width 2) (layer F.Cu) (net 1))
 (segment (start 22.1001 -26.0863) (end 20.2638 -27.9226) (width 2) (layer F.Cu) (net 1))
 (segment (start 22.1001 -24.015) (end 22.1001 -26.0863) (width 2) (layer B.Cu) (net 1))
 (segment (start 22.1001 -26.0863) (end 20.2638 -27.9226) (width 2) (layer B.Cu) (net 1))
 (segment (start 22.1001 -5.985) (end 22.1001 -3.9139) (width 2) (layer B.Cu) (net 7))
 (segment (start 22.1001 -3.9139) (end 20.2638 -2.0776) (width 2) (layer B.Cu) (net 7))
 (segment (start 22.1001 -5.985) (end 22.1001 -3.9139) (width 2) (layer F.Cu) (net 7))
 (segment (start 22.1001 -3.9139) (end 20.2638 -2.0776) (width 2) (layer F.Cu) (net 7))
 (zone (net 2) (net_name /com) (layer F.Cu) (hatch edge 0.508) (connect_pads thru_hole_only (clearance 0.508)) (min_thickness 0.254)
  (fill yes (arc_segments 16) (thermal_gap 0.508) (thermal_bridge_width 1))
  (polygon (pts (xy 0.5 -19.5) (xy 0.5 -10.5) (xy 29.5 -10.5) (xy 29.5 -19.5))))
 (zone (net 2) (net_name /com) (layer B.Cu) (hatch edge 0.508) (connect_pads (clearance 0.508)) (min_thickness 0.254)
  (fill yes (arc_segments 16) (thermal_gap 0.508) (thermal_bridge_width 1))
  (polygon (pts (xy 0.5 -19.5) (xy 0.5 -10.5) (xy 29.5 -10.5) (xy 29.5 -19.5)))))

